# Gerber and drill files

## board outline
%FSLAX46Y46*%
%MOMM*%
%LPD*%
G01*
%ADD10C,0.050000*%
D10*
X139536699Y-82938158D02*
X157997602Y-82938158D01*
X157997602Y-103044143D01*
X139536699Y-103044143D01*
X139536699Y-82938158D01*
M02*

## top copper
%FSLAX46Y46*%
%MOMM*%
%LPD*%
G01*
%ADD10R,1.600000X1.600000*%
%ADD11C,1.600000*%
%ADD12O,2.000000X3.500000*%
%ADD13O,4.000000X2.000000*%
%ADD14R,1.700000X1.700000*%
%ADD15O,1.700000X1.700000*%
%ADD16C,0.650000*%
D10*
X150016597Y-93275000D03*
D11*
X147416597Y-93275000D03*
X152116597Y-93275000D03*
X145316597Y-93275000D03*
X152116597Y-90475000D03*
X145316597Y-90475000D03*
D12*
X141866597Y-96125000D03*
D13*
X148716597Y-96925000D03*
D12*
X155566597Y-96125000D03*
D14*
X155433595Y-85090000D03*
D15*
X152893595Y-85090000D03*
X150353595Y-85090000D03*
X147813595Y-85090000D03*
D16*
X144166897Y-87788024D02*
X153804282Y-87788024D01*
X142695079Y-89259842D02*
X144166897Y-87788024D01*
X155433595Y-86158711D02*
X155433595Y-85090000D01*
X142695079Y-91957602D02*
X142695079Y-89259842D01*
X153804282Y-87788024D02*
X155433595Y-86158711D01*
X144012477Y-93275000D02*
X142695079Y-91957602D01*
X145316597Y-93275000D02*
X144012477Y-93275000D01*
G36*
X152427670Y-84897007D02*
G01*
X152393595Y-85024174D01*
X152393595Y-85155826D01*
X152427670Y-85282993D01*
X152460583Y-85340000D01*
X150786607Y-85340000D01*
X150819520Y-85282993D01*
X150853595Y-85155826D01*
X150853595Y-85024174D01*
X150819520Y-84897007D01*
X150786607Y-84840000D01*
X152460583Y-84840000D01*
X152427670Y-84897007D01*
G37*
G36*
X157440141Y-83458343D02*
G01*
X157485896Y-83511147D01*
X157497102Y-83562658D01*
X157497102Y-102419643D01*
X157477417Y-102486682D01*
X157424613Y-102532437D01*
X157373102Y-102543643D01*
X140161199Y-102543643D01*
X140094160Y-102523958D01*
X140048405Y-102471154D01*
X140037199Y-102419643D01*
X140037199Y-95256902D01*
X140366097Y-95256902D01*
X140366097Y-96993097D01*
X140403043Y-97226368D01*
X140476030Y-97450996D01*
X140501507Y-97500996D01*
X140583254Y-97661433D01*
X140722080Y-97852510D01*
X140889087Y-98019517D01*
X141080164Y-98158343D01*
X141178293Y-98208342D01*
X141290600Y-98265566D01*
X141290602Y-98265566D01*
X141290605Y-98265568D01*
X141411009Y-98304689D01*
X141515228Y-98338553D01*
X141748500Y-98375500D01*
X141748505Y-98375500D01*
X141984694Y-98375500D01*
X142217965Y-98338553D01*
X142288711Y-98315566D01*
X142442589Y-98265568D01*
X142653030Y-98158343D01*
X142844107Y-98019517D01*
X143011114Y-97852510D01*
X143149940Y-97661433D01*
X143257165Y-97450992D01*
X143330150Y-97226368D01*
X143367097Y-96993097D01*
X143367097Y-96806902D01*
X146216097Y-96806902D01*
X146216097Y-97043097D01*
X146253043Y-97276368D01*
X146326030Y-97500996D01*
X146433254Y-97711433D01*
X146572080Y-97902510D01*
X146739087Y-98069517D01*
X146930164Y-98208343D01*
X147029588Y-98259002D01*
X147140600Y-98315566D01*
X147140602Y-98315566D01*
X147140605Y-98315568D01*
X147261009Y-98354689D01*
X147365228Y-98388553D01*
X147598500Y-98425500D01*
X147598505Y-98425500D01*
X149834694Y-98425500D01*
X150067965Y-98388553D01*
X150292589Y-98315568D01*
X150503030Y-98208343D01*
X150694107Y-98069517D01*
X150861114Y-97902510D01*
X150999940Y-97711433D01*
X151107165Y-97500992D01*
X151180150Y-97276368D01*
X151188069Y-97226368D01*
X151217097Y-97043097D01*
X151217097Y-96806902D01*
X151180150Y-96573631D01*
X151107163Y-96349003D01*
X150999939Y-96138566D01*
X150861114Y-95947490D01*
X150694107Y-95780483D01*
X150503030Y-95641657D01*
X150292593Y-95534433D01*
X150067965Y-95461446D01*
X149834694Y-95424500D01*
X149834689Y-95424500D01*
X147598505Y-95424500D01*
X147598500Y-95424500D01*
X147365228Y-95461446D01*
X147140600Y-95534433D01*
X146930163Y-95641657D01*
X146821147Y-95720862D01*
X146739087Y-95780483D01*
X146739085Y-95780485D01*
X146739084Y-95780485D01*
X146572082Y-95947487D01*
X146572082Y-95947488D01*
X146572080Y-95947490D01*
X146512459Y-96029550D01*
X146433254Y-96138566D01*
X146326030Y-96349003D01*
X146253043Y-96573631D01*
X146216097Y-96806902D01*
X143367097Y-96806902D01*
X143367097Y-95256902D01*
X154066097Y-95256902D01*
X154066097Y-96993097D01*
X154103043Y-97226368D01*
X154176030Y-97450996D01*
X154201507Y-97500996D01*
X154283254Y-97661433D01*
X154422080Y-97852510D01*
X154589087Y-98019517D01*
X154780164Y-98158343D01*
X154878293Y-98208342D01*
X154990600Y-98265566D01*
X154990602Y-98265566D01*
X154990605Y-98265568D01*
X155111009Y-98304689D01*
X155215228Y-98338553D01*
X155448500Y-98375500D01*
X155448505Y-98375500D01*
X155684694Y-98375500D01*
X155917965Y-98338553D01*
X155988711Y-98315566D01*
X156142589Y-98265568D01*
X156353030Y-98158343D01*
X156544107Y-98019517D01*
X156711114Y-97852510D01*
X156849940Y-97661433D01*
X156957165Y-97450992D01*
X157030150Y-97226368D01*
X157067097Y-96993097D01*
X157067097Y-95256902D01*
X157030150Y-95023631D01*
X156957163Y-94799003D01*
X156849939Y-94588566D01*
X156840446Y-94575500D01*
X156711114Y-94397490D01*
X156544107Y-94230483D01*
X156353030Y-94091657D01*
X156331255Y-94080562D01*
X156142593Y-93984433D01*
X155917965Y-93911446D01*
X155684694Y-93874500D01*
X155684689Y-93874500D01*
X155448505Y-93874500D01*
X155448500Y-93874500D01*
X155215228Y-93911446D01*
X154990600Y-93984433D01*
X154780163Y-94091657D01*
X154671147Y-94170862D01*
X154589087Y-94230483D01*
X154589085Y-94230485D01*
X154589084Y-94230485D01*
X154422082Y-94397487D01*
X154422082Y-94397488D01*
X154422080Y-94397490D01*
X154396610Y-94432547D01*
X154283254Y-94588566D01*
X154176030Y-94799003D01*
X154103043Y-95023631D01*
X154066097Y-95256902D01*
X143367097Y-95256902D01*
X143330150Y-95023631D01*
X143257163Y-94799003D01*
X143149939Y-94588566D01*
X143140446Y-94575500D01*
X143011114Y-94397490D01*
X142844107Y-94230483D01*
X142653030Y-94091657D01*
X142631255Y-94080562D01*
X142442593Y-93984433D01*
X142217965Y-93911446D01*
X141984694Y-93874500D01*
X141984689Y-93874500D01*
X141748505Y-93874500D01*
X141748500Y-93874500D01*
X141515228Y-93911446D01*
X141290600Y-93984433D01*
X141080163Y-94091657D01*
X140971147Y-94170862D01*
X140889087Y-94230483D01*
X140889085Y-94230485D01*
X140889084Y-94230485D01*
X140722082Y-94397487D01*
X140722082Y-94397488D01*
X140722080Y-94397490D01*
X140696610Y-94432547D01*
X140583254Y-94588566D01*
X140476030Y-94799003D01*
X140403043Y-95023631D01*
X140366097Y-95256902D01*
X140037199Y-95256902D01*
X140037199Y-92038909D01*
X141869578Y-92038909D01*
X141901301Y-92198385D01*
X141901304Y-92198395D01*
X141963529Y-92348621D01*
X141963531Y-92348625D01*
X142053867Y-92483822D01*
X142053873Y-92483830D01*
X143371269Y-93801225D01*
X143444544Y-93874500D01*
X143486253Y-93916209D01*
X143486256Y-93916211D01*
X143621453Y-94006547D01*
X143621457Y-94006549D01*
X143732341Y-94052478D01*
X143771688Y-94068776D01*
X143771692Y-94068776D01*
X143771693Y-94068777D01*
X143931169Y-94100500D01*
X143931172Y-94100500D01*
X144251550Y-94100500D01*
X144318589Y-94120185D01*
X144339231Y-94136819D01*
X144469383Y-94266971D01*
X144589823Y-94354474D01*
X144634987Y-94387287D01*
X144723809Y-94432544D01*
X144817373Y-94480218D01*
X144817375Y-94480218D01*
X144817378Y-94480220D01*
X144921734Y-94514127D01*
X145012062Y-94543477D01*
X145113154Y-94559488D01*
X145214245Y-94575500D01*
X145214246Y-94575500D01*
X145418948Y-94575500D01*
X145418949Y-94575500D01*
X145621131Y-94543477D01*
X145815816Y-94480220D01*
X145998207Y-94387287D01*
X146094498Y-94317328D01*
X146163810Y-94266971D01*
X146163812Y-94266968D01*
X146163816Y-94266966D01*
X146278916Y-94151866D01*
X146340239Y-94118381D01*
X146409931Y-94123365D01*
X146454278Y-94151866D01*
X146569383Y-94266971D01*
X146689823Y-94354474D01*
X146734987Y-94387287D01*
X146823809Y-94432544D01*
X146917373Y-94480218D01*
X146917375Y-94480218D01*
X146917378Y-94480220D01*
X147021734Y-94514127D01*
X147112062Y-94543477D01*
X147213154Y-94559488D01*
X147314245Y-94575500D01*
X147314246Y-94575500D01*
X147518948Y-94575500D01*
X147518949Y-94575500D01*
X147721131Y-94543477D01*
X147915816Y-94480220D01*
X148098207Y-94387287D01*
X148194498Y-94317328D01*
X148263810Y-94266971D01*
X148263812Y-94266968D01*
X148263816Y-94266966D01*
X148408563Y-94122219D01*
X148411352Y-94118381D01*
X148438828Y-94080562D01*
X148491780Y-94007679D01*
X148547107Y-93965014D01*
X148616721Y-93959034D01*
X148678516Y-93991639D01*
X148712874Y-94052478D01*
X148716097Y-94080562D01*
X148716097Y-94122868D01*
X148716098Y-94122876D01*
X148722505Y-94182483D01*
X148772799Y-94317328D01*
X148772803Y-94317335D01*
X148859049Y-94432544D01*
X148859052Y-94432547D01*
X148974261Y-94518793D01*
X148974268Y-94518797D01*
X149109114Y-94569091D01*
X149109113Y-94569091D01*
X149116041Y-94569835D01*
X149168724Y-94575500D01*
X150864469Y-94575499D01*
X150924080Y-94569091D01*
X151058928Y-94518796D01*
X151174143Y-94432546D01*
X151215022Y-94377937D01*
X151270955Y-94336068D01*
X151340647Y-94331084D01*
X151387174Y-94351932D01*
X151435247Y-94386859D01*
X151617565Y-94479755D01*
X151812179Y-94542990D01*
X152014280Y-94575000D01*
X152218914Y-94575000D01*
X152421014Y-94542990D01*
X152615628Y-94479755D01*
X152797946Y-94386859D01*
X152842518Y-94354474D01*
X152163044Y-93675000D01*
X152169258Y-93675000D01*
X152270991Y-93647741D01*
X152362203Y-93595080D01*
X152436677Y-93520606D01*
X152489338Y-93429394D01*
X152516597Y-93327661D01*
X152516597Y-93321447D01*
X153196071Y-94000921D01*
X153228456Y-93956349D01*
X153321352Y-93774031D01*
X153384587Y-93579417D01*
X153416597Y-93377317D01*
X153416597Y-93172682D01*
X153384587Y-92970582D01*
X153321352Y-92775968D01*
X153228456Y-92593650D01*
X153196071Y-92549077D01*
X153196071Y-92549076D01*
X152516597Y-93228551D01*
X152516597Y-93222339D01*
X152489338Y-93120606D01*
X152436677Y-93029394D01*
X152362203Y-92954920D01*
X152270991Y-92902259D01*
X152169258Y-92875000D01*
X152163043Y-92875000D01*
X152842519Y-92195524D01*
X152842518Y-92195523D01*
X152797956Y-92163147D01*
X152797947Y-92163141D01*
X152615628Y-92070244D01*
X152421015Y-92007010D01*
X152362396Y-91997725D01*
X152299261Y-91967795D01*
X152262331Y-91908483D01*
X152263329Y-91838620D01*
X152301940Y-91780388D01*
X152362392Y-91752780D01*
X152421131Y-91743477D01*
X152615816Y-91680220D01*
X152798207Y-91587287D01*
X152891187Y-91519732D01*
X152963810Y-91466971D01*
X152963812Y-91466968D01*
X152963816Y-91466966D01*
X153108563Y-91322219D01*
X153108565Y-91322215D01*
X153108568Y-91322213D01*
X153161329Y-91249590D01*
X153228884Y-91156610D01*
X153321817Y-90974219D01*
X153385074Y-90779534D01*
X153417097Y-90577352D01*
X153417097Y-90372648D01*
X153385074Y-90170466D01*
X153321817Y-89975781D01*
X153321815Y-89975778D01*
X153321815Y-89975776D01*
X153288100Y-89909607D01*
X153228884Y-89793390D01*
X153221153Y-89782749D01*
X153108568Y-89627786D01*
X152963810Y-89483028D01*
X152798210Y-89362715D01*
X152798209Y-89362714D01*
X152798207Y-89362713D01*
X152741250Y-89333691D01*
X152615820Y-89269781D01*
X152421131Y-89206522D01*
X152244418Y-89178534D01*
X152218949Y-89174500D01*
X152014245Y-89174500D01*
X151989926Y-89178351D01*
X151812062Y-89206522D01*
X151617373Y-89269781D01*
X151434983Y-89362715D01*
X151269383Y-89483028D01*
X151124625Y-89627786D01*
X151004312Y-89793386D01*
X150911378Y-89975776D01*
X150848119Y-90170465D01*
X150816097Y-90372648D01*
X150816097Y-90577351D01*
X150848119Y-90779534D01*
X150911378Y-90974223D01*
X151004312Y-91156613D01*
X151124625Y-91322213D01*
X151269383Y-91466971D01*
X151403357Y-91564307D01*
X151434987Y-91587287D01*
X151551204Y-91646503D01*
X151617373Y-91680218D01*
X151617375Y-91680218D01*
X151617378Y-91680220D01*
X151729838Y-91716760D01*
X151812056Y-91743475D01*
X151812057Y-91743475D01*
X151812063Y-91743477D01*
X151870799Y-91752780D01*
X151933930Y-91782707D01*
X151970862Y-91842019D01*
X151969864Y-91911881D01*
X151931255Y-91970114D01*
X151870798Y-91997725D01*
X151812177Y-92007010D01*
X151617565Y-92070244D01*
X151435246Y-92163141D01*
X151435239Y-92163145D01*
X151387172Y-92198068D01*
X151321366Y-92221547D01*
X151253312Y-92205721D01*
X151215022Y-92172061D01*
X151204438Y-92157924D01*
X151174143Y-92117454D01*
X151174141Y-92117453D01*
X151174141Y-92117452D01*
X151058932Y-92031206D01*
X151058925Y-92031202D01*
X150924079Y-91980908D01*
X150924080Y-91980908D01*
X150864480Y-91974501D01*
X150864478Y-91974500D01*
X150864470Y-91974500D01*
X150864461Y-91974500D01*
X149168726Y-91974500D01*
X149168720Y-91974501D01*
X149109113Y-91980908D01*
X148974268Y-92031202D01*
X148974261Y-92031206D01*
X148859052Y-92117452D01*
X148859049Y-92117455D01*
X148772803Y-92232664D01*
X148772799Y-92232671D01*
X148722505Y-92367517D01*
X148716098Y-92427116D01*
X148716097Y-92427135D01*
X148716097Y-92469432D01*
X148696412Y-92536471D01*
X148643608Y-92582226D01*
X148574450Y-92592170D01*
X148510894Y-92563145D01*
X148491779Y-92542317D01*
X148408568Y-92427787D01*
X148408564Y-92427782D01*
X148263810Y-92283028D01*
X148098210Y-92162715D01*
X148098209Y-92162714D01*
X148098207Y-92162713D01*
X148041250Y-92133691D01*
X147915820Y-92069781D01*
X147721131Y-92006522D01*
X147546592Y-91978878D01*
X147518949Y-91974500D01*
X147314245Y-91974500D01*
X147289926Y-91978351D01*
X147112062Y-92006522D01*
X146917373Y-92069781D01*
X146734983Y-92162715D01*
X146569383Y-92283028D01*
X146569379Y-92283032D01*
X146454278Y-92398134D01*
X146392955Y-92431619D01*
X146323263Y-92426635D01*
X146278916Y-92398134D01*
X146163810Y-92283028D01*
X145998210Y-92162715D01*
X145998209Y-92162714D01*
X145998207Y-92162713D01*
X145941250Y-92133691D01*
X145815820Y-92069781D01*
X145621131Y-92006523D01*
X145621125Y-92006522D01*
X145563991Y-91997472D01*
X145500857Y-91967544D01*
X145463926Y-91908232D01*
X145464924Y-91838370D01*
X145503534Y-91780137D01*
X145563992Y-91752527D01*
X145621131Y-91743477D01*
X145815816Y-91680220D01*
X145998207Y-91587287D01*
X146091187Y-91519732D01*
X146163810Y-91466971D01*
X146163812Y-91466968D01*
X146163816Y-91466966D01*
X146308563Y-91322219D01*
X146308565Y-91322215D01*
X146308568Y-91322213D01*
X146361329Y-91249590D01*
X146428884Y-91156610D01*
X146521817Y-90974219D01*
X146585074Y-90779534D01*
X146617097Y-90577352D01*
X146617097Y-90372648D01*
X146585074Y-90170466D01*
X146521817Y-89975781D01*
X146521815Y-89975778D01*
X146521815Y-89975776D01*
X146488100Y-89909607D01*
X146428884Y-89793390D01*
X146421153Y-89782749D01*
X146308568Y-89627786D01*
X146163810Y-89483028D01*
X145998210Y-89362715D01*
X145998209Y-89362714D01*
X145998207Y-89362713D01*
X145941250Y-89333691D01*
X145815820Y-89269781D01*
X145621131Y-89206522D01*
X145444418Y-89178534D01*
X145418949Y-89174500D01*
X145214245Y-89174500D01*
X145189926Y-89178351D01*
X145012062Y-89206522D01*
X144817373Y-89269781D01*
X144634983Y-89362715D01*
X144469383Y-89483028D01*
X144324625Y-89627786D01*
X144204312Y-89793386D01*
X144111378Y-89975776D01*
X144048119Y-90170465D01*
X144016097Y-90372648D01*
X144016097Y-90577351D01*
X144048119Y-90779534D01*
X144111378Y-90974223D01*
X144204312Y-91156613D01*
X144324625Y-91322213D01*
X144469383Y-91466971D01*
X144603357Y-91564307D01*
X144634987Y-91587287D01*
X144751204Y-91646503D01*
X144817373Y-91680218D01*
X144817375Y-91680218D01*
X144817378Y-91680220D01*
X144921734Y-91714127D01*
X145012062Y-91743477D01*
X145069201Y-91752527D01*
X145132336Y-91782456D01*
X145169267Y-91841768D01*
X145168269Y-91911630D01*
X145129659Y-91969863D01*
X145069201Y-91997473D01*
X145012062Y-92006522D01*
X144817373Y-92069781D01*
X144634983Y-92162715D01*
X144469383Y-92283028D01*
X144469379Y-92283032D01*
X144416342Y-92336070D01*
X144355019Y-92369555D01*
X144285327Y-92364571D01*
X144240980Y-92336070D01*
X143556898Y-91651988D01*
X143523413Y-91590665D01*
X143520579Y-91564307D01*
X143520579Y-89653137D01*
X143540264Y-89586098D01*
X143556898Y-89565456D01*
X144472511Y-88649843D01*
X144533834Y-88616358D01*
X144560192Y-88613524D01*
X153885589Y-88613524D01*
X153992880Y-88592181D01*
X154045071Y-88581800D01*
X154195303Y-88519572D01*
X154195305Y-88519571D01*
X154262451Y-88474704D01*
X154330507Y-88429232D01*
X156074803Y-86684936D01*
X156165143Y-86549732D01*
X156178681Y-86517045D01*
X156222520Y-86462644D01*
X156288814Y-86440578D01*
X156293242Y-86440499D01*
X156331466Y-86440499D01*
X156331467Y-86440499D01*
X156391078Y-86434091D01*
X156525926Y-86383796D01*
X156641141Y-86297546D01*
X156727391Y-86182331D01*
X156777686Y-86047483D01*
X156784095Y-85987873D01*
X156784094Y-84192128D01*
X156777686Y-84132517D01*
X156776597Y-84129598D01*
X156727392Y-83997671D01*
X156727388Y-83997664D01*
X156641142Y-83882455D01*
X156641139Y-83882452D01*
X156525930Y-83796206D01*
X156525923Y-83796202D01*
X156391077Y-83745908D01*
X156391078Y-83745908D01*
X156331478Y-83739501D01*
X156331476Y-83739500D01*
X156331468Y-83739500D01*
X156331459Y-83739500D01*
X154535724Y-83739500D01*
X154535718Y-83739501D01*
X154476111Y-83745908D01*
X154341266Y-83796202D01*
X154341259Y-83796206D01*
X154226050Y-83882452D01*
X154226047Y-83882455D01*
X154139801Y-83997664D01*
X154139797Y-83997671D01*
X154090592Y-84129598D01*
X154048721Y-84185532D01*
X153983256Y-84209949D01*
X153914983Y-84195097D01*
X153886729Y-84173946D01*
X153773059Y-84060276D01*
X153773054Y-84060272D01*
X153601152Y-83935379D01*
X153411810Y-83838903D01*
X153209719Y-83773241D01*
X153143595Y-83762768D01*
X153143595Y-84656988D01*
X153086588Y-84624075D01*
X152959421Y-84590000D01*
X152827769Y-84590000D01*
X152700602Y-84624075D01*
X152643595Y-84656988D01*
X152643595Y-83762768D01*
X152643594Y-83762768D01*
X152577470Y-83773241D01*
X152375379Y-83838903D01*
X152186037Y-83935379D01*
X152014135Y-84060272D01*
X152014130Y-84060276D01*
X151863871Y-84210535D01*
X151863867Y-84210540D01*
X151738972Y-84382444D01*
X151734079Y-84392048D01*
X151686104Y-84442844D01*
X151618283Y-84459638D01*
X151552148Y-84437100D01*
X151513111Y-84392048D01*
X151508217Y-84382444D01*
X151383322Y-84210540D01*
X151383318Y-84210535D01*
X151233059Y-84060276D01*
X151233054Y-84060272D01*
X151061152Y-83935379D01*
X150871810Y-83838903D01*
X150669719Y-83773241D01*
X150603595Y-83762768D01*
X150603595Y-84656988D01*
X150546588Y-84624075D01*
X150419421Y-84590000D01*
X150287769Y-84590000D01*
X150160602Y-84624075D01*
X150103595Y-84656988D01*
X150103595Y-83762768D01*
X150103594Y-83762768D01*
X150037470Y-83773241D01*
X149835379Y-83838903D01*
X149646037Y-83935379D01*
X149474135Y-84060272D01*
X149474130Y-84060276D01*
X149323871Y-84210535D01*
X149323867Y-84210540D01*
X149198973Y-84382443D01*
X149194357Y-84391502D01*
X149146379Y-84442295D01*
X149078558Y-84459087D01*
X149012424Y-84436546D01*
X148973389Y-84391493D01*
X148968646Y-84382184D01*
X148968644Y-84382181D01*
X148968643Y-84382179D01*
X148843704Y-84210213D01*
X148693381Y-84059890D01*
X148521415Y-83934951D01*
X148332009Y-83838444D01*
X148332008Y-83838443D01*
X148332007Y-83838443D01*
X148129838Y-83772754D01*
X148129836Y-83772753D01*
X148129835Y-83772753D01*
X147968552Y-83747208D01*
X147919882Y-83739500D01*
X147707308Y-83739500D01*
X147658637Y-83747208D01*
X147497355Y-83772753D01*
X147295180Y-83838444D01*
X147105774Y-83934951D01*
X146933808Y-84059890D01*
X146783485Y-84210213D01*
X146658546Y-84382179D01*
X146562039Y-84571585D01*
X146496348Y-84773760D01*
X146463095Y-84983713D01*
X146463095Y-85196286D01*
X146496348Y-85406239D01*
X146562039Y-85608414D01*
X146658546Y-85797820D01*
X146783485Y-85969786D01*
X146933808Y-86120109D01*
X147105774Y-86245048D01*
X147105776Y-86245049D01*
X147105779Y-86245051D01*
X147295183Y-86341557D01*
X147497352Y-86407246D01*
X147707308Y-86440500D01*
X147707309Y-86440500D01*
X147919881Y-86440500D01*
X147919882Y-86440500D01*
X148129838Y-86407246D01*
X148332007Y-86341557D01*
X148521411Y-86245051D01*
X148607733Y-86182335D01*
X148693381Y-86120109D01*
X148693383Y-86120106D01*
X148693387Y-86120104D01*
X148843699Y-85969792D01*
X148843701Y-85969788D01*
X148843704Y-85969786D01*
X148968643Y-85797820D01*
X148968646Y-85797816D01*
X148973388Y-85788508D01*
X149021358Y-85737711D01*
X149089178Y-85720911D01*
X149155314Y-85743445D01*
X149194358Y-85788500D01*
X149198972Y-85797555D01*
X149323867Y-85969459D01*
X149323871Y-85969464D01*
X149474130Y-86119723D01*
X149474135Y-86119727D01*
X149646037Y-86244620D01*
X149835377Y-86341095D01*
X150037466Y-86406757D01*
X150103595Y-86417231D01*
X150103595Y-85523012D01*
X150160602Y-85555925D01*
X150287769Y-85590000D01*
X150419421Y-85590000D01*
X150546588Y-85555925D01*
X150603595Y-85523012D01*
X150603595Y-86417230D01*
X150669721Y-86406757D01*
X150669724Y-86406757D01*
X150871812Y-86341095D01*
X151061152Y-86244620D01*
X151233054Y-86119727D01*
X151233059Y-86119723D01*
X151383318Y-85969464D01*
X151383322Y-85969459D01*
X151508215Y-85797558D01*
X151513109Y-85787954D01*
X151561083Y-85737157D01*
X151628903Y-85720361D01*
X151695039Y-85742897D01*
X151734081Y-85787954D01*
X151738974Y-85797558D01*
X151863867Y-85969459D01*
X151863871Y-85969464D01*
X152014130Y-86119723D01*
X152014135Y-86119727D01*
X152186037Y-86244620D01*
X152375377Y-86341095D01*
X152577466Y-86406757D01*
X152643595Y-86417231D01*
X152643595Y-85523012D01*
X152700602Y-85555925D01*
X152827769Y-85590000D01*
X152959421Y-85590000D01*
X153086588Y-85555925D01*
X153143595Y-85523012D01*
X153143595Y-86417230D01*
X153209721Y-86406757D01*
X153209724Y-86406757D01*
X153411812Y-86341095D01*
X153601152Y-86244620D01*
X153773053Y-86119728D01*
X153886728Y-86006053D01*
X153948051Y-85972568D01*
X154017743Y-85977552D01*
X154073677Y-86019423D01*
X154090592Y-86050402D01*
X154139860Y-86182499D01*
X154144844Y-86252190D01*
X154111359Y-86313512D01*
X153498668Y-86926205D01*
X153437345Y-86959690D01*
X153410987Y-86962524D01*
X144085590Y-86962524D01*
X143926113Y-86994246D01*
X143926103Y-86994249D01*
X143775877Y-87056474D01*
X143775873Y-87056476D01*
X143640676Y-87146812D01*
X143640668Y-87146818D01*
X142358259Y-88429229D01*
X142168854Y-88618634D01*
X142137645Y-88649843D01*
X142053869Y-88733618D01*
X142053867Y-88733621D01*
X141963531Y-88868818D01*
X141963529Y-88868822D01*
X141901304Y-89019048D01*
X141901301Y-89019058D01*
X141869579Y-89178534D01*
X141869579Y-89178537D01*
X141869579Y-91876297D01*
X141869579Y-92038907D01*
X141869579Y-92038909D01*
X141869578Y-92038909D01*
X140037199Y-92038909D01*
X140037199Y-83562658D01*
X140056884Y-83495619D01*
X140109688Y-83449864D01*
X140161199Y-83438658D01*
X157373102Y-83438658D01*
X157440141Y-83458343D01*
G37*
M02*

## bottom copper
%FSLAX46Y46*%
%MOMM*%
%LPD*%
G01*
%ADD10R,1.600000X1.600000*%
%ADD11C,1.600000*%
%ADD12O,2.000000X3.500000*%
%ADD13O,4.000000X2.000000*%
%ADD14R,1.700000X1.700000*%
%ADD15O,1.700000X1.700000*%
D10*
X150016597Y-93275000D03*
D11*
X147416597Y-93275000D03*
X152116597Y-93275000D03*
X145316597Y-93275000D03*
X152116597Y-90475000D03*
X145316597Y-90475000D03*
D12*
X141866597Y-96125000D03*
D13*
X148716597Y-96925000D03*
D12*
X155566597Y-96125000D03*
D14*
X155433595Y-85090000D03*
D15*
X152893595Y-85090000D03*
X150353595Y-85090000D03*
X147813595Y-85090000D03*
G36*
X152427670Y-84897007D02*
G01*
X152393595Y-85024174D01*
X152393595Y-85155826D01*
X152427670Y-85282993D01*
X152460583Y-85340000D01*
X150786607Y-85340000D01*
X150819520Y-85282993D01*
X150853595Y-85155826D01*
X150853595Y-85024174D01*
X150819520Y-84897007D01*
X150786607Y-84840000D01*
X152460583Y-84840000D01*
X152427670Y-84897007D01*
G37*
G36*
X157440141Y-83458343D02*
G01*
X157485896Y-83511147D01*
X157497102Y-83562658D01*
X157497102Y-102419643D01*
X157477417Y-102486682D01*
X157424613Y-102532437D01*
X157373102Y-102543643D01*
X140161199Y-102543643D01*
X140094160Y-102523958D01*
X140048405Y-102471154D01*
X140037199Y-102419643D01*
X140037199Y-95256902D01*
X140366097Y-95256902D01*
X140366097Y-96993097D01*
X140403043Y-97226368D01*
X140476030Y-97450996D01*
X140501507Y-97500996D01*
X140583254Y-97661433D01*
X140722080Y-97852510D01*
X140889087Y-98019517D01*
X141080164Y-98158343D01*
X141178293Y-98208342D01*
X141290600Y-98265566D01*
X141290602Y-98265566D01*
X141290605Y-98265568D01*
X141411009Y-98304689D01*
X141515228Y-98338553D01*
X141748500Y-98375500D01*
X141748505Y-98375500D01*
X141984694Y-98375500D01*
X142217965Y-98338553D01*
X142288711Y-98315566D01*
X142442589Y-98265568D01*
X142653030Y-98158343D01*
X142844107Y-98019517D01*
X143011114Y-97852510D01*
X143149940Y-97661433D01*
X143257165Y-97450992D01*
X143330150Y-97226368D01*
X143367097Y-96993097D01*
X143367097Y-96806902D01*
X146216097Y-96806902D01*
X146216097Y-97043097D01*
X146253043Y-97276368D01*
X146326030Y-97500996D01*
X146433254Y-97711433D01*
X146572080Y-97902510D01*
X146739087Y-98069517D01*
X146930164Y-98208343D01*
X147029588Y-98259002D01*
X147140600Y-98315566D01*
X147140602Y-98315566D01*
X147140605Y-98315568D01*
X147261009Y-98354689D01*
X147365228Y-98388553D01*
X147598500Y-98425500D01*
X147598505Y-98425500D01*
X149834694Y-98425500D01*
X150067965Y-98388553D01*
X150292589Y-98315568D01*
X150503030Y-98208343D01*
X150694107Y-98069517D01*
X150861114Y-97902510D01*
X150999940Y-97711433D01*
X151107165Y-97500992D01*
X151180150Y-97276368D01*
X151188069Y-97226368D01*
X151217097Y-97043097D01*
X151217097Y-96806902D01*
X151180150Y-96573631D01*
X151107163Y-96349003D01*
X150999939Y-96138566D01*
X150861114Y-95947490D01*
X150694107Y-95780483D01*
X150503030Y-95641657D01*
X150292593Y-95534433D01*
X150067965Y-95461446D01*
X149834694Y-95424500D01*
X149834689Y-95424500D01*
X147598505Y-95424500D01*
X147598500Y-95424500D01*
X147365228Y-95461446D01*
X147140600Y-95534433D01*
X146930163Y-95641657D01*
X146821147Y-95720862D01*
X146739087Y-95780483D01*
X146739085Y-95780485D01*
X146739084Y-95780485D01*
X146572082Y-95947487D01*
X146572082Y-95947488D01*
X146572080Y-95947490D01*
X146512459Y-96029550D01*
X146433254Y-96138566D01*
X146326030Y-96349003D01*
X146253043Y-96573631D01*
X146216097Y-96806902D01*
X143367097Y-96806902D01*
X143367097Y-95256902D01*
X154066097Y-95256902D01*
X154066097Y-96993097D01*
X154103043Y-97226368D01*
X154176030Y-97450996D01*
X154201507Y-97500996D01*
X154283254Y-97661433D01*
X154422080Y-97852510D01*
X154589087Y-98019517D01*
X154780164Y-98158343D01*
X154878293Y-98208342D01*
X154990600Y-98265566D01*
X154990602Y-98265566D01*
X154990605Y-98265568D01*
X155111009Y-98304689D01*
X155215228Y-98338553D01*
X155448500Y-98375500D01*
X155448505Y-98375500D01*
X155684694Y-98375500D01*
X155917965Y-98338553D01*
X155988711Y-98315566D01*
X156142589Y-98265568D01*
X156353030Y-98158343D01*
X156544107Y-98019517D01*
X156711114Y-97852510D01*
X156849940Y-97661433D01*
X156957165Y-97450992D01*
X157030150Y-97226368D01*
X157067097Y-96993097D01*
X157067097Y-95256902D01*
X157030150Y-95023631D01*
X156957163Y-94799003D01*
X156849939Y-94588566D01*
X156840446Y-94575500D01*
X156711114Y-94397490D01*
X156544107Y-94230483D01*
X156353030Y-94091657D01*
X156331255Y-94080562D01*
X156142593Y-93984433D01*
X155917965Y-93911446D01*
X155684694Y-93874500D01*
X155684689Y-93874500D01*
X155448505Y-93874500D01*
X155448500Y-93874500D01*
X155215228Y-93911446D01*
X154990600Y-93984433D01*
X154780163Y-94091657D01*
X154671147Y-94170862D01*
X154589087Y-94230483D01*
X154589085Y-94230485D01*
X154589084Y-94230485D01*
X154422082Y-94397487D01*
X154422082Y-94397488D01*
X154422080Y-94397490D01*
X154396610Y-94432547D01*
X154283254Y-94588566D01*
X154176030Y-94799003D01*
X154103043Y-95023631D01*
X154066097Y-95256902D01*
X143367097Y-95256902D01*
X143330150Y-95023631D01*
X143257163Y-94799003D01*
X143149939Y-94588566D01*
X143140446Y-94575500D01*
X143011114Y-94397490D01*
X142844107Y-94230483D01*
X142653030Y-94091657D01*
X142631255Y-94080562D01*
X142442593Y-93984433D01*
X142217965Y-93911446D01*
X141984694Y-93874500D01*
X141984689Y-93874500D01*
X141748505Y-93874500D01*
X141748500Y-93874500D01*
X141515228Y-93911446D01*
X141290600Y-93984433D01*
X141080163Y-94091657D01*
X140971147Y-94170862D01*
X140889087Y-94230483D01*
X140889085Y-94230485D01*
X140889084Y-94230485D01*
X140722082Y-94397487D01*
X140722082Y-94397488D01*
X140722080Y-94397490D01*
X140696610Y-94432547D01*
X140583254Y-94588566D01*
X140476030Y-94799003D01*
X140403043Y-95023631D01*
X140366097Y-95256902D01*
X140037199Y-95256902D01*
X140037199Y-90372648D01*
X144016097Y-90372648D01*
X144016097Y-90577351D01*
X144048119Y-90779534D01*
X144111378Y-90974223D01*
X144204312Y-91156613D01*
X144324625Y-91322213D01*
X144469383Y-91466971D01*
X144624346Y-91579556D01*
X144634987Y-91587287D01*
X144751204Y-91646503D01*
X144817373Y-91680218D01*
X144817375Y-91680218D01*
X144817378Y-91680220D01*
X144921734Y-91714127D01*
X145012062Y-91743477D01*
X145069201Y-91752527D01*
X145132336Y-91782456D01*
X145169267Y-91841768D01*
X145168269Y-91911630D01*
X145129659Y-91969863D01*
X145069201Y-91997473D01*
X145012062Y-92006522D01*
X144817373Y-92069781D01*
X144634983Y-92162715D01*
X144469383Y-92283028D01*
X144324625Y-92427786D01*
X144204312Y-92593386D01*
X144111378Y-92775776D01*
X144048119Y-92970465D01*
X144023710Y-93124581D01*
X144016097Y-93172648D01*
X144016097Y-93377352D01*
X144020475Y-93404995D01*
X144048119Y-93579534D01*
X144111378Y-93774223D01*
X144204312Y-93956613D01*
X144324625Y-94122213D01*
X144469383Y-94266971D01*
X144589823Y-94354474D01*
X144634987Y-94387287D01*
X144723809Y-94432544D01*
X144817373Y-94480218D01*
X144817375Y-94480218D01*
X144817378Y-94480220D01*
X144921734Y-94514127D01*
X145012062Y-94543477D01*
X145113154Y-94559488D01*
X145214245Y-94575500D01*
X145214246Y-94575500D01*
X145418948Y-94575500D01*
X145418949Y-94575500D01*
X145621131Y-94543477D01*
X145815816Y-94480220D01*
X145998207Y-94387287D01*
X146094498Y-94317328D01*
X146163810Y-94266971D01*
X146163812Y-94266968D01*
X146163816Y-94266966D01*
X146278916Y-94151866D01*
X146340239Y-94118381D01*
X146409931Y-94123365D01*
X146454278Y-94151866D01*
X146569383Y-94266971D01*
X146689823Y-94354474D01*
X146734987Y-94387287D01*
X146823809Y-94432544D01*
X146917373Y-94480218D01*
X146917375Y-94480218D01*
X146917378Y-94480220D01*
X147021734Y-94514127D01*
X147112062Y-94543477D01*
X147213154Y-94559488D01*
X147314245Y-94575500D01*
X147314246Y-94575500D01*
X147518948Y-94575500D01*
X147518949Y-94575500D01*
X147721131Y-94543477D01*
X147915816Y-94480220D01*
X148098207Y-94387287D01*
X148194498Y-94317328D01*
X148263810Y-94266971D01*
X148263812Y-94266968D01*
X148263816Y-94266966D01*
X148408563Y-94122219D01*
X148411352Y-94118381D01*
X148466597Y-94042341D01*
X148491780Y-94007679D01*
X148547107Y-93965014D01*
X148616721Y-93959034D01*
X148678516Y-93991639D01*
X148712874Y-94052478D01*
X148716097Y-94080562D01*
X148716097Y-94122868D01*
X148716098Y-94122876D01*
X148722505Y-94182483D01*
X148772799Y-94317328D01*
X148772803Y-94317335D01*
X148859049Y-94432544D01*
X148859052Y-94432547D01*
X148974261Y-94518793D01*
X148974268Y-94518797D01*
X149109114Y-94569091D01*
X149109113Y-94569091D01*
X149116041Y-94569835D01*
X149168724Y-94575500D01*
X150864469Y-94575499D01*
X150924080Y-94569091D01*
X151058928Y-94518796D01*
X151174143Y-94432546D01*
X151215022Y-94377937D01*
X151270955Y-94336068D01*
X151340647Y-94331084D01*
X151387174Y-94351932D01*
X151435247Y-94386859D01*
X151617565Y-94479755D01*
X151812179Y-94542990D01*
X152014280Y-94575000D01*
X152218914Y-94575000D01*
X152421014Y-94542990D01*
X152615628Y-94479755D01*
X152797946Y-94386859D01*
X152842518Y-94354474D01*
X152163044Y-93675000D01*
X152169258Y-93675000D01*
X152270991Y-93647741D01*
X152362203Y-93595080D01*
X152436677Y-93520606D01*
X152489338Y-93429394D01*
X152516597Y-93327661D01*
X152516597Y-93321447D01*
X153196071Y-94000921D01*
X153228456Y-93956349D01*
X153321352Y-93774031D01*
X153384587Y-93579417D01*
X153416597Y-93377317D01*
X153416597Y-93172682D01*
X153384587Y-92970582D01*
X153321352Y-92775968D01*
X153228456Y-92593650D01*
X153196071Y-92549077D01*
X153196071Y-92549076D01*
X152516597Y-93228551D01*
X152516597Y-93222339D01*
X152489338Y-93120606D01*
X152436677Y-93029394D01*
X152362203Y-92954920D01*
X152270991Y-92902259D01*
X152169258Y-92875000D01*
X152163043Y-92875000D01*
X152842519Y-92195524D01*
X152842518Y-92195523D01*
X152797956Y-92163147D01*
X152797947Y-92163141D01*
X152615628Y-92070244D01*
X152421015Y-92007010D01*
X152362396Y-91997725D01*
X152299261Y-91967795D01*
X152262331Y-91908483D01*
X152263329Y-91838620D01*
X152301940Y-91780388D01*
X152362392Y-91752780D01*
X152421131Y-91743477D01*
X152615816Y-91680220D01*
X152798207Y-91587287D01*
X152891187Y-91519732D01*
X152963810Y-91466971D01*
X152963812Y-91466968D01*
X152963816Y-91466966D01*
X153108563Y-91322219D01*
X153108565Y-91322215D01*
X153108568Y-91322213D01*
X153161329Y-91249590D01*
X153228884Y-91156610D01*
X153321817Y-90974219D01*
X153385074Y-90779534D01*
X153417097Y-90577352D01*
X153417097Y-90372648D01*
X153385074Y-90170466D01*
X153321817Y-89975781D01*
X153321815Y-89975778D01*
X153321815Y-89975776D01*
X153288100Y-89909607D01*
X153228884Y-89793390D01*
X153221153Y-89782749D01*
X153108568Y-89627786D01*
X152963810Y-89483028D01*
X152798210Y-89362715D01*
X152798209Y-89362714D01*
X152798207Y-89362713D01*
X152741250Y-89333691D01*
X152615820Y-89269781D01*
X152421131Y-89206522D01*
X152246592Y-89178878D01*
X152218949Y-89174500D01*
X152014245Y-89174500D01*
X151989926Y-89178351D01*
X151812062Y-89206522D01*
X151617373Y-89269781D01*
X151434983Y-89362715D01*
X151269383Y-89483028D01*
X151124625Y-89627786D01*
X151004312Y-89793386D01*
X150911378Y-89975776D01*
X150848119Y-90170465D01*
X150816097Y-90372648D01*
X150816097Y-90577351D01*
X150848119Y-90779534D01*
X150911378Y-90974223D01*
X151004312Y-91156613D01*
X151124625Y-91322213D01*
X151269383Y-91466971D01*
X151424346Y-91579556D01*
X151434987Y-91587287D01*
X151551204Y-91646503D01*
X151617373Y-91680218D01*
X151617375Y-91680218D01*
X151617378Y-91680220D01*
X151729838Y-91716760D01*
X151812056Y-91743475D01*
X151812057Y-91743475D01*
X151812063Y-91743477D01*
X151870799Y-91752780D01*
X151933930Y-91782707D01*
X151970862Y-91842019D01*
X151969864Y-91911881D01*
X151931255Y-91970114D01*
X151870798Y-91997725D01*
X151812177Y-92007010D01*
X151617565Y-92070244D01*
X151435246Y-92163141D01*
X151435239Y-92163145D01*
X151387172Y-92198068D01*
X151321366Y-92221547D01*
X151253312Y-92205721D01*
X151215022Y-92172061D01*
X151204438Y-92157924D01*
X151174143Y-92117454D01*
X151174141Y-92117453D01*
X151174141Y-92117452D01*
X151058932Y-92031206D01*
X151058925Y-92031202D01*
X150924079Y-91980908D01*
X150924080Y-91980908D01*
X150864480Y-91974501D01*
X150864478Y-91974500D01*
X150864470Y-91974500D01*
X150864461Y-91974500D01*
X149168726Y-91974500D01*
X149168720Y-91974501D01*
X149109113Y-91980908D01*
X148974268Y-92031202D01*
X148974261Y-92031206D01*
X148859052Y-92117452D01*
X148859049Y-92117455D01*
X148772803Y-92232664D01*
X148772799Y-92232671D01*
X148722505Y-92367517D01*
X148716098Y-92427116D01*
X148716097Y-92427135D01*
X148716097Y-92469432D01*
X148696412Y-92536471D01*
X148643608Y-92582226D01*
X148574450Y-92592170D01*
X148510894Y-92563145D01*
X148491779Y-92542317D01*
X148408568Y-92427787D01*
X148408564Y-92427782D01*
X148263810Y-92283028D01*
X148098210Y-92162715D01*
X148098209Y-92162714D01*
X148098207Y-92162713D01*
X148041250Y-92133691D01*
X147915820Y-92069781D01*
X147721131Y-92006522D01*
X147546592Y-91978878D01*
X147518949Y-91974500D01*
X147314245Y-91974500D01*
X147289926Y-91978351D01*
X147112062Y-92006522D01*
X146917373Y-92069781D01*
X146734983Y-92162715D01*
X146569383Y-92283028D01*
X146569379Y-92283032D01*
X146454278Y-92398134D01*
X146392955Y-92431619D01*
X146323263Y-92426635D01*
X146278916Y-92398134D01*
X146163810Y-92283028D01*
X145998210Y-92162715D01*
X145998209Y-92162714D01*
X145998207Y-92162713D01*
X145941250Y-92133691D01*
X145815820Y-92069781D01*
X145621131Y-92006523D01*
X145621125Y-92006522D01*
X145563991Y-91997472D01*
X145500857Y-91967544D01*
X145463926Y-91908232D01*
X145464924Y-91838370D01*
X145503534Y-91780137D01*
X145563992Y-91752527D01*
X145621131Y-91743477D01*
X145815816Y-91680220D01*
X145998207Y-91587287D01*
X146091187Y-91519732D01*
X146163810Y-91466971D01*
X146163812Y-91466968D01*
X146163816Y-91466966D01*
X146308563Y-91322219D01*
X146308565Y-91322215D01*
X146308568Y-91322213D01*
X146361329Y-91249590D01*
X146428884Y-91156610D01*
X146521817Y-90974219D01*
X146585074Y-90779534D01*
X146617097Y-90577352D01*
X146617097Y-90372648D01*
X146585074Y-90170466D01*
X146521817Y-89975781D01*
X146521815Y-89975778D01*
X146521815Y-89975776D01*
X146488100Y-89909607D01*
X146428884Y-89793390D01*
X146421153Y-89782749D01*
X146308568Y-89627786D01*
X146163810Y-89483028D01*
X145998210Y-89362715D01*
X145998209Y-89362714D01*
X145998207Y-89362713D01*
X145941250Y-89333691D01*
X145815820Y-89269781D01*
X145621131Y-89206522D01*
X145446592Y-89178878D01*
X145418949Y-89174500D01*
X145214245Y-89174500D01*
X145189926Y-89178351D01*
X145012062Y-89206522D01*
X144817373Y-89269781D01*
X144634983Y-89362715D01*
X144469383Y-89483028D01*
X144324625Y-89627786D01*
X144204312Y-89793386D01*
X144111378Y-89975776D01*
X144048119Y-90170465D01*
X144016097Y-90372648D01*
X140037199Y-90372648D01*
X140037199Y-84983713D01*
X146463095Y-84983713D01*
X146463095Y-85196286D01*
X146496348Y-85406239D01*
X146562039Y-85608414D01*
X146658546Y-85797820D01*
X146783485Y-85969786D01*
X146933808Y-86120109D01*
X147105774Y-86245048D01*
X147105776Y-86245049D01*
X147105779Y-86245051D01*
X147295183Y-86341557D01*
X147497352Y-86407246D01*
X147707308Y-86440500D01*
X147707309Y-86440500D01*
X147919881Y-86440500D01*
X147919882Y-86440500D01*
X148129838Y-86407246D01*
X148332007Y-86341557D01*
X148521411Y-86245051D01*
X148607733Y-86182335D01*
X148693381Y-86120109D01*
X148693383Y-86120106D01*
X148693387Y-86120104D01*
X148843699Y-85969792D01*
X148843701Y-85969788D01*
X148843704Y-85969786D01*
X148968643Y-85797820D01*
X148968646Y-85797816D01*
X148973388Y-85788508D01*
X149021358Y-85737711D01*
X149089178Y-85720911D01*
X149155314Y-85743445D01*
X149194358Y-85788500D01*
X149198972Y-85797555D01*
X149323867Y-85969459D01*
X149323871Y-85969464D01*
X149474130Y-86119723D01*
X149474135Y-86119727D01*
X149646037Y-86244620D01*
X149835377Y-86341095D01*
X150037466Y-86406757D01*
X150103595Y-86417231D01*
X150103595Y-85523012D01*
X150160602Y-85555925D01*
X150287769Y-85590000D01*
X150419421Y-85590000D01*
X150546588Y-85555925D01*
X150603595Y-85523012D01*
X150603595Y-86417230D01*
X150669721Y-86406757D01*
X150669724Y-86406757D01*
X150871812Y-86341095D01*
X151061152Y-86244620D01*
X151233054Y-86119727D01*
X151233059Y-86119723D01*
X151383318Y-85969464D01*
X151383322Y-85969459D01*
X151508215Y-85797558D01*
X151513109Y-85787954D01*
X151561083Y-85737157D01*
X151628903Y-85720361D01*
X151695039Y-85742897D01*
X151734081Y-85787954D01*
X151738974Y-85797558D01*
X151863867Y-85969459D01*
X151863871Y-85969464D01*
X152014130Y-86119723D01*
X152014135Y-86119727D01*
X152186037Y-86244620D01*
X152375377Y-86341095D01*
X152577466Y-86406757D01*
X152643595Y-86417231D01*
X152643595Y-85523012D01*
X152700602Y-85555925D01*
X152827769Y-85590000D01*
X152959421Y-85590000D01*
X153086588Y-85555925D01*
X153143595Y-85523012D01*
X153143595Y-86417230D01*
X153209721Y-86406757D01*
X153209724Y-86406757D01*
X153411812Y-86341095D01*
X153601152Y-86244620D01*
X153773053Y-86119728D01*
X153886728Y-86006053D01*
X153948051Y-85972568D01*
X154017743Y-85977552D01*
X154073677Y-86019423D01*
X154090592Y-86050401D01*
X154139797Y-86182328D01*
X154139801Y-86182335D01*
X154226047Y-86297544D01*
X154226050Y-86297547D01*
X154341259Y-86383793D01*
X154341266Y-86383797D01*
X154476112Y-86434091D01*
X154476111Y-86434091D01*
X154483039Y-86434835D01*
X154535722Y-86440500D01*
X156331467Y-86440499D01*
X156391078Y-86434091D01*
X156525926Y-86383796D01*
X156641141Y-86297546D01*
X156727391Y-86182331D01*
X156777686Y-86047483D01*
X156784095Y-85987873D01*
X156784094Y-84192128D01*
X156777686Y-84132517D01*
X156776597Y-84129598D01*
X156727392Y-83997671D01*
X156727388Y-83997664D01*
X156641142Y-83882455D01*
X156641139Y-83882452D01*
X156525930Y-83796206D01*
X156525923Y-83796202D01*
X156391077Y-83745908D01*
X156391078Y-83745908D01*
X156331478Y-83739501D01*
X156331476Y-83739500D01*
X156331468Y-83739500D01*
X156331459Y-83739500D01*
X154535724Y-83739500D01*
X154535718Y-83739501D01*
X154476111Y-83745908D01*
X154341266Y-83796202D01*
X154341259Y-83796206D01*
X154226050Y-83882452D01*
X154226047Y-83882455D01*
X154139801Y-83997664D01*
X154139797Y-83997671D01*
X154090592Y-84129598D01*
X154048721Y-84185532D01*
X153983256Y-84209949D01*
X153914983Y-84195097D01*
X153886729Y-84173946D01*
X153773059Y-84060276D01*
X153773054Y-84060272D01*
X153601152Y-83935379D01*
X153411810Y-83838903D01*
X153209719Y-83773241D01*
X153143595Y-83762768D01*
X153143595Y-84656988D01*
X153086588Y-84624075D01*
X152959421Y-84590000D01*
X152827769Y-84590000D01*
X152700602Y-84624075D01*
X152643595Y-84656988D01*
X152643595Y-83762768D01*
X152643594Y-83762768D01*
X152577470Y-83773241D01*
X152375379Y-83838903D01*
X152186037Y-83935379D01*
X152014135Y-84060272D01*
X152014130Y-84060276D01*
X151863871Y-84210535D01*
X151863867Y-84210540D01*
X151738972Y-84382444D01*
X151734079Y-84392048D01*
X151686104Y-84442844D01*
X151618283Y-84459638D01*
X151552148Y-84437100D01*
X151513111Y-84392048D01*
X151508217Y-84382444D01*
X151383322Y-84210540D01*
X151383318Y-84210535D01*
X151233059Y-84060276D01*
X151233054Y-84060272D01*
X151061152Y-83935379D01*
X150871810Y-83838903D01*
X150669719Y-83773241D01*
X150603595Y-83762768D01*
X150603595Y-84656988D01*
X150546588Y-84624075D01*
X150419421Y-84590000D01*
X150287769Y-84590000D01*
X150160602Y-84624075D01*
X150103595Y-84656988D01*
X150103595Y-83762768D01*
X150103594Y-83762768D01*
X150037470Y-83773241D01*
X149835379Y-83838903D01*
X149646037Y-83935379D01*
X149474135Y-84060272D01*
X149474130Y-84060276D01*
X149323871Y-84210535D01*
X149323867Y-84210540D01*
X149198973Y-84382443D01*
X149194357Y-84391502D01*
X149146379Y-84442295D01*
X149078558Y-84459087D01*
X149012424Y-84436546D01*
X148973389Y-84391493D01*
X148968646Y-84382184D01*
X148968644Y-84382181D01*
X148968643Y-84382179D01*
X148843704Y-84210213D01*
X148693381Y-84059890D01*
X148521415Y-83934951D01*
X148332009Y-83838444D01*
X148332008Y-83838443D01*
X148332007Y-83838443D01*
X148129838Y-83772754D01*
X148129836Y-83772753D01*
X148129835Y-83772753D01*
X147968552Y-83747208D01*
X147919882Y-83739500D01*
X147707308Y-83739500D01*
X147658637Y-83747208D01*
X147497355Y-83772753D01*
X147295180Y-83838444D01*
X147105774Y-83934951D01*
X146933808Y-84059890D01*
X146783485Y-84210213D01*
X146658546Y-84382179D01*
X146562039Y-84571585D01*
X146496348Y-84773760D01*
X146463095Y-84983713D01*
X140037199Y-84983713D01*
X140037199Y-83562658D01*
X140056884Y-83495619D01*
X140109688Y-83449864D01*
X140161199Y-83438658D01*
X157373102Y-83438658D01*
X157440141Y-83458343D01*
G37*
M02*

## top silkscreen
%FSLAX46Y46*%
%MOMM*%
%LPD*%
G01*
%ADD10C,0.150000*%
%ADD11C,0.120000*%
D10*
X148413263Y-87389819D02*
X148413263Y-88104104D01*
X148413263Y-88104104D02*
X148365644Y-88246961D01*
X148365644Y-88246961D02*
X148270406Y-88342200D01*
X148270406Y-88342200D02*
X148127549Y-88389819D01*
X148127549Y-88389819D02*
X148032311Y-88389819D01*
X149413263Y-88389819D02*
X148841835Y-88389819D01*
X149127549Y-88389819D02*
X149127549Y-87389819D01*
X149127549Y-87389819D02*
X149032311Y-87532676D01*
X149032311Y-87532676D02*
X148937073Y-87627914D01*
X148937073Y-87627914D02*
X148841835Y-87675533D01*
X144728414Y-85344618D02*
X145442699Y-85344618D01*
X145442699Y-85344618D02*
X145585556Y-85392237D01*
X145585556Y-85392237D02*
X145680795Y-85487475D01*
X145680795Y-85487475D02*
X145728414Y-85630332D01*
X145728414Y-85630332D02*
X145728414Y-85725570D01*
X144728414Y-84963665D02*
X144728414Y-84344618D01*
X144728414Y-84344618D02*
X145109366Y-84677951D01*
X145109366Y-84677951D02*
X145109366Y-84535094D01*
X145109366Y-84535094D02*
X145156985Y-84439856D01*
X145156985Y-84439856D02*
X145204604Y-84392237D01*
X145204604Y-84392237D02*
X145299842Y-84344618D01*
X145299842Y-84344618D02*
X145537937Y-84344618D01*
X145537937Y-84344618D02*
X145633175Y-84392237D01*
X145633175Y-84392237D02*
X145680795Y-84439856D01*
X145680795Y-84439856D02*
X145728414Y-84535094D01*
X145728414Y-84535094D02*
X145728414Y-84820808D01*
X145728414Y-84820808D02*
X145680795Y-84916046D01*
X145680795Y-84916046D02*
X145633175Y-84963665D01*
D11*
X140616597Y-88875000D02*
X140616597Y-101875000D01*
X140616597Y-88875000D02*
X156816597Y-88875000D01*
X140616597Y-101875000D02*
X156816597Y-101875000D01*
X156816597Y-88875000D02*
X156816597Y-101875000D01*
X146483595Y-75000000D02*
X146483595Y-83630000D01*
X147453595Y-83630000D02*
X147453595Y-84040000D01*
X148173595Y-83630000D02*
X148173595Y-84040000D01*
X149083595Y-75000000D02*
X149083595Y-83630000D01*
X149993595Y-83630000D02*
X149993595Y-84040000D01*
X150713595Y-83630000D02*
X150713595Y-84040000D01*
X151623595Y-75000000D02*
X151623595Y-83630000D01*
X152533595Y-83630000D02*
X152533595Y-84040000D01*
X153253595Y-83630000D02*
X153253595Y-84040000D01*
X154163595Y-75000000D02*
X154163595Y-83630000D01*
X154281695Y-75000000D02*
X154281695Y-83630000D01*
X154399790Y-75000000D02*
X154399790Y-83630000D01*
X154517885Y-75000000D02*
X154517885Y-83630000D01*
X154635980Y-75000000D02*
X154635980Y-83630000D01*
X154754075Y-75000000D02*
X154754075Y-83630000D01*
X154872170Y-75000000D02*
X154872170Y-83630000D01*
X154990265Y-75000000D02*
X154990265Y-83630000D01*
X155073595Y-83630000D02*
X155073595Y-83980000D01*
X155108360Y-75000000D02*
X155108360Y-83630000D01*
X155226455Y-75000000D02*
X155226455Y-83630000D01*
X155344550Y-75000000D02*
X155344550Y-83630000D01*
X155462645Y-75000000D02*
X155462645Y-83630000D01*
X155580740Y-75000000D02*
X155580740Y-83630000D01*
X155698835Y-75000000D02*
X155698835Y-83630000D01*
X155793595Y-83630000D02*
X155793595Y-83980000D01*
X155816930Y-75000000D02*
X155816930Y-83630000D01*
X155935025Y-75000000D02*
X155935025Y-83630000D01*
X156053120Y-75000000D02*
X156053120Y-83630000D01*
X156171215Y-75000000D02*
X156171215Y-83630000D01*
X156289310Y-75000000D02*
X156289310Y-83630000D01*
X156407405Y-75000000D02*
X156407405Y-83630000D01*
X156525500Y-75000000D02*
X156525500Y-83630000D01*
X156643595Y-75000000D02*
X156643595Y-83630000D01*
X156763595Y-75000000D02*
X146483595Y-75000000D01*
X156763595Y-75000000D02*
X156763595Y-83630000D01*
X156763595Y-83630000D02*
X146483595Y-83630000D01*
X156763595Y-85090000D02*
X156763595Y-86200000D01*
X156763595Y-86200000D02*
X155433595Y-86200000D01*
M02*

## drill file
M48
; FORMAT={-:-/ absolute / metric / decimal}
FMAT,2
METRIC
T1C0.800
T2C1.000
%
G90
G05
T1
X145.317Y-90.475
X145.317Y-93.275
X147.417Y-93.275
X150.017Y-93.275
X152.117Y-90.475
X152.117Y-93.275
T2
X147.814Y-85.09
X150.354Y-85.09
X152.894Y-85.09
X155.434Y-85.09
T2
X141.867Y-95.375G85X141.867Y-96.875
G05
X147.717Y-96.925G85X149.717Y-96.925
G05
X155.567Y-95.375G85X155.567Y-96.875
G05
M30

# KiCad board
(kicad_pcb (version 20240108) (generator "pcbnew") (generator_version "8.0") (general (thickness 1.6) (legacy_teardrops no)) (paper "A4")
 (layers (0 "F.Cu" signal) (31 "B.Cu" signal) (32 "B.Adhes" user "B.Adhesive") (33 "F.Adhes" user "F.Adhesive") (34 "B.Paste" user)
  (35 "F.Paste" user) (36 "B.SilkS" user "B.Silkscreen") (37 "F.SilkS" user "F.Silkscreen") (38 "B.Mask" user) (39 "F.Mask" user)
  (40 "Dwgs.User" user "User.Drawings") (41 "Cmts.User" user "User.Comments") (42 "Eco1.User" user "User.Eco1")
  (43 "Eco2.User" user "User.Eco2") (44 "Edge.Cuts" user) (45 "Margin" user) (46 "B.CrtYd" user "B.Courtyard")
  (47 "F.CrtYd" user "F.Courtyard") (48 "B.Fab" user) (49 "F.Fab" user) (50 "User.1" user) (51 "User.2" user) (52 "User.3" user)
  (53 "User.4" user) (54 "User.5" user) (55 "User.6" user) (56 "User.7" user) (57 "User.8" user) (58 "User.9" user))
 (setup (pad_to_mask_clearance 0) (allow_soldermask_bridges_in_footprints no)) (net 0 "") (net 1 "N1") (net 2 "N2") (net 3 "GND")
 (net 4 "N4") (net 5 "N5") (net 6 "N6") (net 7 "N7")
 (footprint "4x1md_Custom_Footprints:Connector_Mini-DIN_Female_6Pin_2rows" (layer "F.Cu") (at 150.016597 93.275)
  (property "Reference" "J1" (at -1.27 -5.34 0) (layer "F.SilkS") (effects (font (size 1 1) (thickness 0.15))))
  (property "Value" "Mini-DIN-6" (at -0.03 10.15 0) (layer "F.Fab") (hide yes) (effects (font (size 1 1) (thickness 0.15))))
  (fp_line (start -9.4 -4.4) (end -9.4 8.6) (stroke (width 0.12) (type solid)) (layer "F.SilkS"))
  (fp_line (start -9.4 -4.4) (end 6.8 -4.4) (stroke (width 0.12) (type solid)) (layer "F.SilkS"))
  (fp_line (start -9.4 8.6) (end 6.8 8.6) (stroke (width 0.12) (type solid)) (layer "F.SilkS"))
  (fp_line (start 6.8 -4.4) (end 6.8 8.6) (stroke (width 0.12) (type solid)) (layer "F.SilkS"))
  (pad "1" thru_hole rect (at 0 0) (size 1.6 1.6) (drill 0.8) (layers "*.Cu" "*.Mask") (remove_unused_layers no) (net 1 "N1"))
  (pad "2" thru_hole circle (at -2.6 0) (size 1.6 1.6) (drill 0.8) (layers "*.Cu" "*.Mask") (remove_unused_layers no) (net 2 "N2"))
  (pad "3" thru_hole circle (at 2.1 0) (size 1.6 1.6) (drill 0.8) (layers "*.Cu" "*.Mask") (remove_unused_layers no) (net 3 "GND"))
  (pad "4" thru_hole circle (at -4.7 0) (size 1.6 1.6) (drill 0.8) (layers "*.Cu" "*.Mask") (remove_unused_layers no) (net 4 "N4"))
  (pad "5" thru_hole circle (at 2.1 -2.8) (size 1.6 1.6) (drill 0.8) (layers "*.Cu" "*.Mask") (remove_unused_layers no) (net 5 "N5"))
  (pad "6" thru_hole circle (at -4.7 -2.8) (size 1.6 1.6) (drill 0.8) (layers "*.Cu" "*.Mask") (remove_unused_layers no) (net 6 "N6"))
  (pad "7" thru_hole oval (at -8.15 2.85) (size 2 3.5) (drill oval 1 2.5) (layers "*.Cu" "*.Mask") (remove_unused_layers no))
  (pad "7" thru_hole oval (at -1.3 3.65) (size 4 2) (drill oval 3 1) (layers "*.Cu" "*.Mask") (remove_unused_layers no))
  (pad "7" thru_hole oval (at 5.55 2.85) (size 2 3.5) (drill oval 1 2.5) (layers "*.Cu" "*.Mask") (remove_unused_layers no)))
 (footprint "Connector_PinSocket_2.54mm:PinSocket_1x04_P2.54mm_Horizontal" (layer "F.Cu") (at 155.433595 85.09 -90)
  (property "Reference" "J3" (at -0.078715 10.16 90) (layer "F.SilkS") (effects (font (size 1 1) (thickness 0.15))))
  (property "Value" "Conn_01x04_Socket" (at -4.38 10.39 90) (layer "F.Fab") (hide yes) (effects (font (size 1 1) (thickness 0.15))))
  (fp_line (start -10.09 8.95) (end -1.46 8.95) (stroke (width 0.12) (type solid)) (layer "F.SilkS"))
  (fp_line (start -1.46 7.98) (end -1.05 7.98) (stroke (width 0.12) (type solid)) (layer "F.SilkS"))
  (fp_line (start -1.46 7.26) (end -1.05 7.26) (stroke (width 0.12) (type solid)) (layer "F.SilkS"))
  (fp_line (start -10.09 6.35) (end -1.46 6.35) (stroke (width 0.12) (type solid)) (layer "F.SilkS"))
  (fp_line (start -1.46 5.44) (end -1.05 5.44) (stroke (width 0.12) (type solid)) (layer "F.SilkS"))
  (fp_line (start -1.46 4.72) (end -1.05 4.72) (stroke (width 0.12) (type solid)) (layer "F.SilkS"))
  (fp_line (start -10.09 3.81) (end -1.46 3.81) (stroke (width 0.12) (type solid)) (layer "F.SilkS"))
  (fp_line (start -1.46 2.9) (end -1.05 2.9) (stroke (width 0.12) (type solid)) (layer "F.SilkS"))
  (fp_line (start -1.46 2.18) (end -1.05 2.18) (stroke (width 0.12) (type solid)) (layer "F.SilkS"))
  (fp_line (start -10.09 1.27) (end -1.46 1.27) (stroke (width 0.12) (type solid)) (layer "F.SilkS"))
  (fp_line (start -10.09 1.1519) (end -1.46 1.1519) (stroke (width 0.12) (type solid)) (layer "F.SilkS"))
  (fp_line (start -10.09 1.033805) (end -1.46 1.033805) (stroke (width 0.12) (type solid)) (layer "F.SilkS"))
  (fp_line (start -10.09 0.91571) (end -1.46 0.91571) (stroke (width 0.12) (type solid)) (layer "F.SilkS"))
  (fp_line (start -10.09 0.797615) (end -1.46 0.797615) (stroke (width 0.12) (type solid)) (layer "F.SilkS"))
  (fp_line (start -10.09 0.67952) (end -1.46 0.67952) (stroke (width 0.12) (type solid)) (layer "F.SilkS"))
  (fp_line (start -10.09 0.561425) (end -1.46 0.561425) (stroke (width 0.12) (type solid)) (layer "F.SilkS"))
  (fp_line (start -10.09 0.44333) (end -1.46 0.44333) (stroke (width 0.12) (type solid)) (layer "F.SilkS"))
  (fp_line (start -1.46 0.36) (end -1.11 0.36) (stroke (width 0.12) (type solid)) (layer "F.SilkS"))
  (fp_line (start -10.09 0.325235) (end -1.46 0.325235) (stroke (width 0.12) (type solid)) (layer "F.SilkS"))
  (fp_line (start -10.09 0.20714) (end -1.46 0.20714) (stroke (width 0.12) (type solid)) (layer "F.SilkS"))
  (fp_line (start -10.09 0.089045) (end -1.46 0.089045) (stroke (width 0.12) (type solid)) (layer "F.SilkS"))
  (fp_line (start -10.09 -0.02905) (end -1.46 -0.02905) (stroke (width 0.12) (type solid)) (layer "F.SilkS"))
  (fp_line (start -10.09 -0.147145) (end -1.46 -0.147145) (stroke (width 0.12) (type solid)) (layer "F.SilkS"))
  (fp_line (start -10.09 -0.26524) (end -1.46 -0.26524) (stroke (width 0.12) (type solid)) (layer "F.SilkS"))
  (fp_line (start -1.46 -0.36) (end -1.11 -0.36) (stroke (width 0.12) (type solid)) (layer "F.SilkS"))
  (fp_line (start -10.09 -0.383335) (end -1.46 -0.383335) (stroke (width 0.12) (type solid)) (layer "F.SilkS"))
  (fp_line (start -10.09 -0.50143) (end -1.46 -0.50143) (stroke (width 0.12) (type solid)) (layer "F.SilkS"))
  (fp_line (start -10.09 -0.619525) (end -1.46 -0.619525) (stroke (width 0.12) (type solid)) (layer "F.SilkS"))
  (fp_line (start -10.09 -0.73762) (end -1.46 -0.73762) (stroke (width 0.12) (type solid)) (layer "F.SilkS"))
  (fp_line (start -10.09 -0.855715) (end -1.46 -0.855715) (stroke (width 0.12) (type solid)) (layer "F.SilkS"))
  (fp_line (start -10.09 -0.97381) (end -1.46 -0.97381) (stroke (width 0.12) (type solid)) (layer "F.SilkS"))
  (fp_line (start -10.09 -1.091905) (end -1.46 -1.091905) (stroke (width 0.12) (type solid)) (layer "F.SilkS"))
  (fp_line (start -10.09 -1.21) (end -1.46 -1.21) (stroke (width 0.12) (type solid)) (layer "F.SilkS"))
  (fp_line (start -10.09 -1.33) (end -10.09 8.95) (stroke (width 0.12) (type solid)) (layer "F.SilkS"))
  (fp_line (start -10.09 -1.33) (end -1.46 -1.33) (stroke (width 0.12) (type solid)) (layer "F.SilkS"))
  (fp_line (start -1.46 -1.33) (end -1.46 8.95) (stroke (width 0.12) (type solid)) (layer "F.SilkS"))
  (fp_line (start 0 -1.33) (end 1.11 -1.33) (stroke (width 0.12) (type solid)) (layer "F.SilkS"))
  (fp_line (start 1.11 -1.33) (end 1.11 0) (stroke (width 0.12) (type solid)) (layer "F.SilkS"))
  (pad "1" thru_hole rect (at 0 0 270) (size 1.7 1.7) (drill 1) (layers "*.Cu" "*.Mask") (remove_unused_layers no) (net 4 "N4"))
  (pad "2" thru_hole oval (at 0 2.54 270) (size 1.7 1.7) (drill 1) (layers "*.Cu" "*.Mask") (remove_unused_layers no) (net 3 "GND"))
  (pad "3" thru_hole oval (at 0 5.08 270) (size 1.7 1.7) (drill 1) (layers "*.Cu" "*.Mask") (remove_unused_layers no) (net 3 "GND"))
  (pad "4" thru_hole oval (at 0 7.62 270) (size 1.7 1.7) (drill 1) (layers "*.Cu" "*.Mask") (remove_unused_layers no) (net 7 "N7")))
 (gr_rect (start 139.536699 82.938158) (end 157.997602 103.044143) (stroke (width 0.05) (type default)) (fill none) (layer "Edge.Cuts"))
 (segment (start 144.166897 87.788024) (end 153.804282 87.788024) (width 0.65) (layer "F.Cu") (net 4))
 (segment (start 142.695079 89.259842) (end 144.166897 87.788024) (width 0.65) (layer "F.Cu") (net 4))
 (segment (start 155.433595 86.158711) (end 155.433595 85.09) (width 0.65) (layer "F.Cu") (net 4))
 (segment (start 142.695079 91.957602) (end 142.695079 89.259842) (width 0.65) (layer "F.Cu") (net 4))
 (segment (start 153.804282 87.788024) (end 155.433595 86.158711) (width 0.65) (layer "F.Cu") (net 4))
 (segment (start 144.012477 93.275) (end 142.695079 91.957602) (width 0.65) (layer "F.Cu") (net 4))
 (segment (start 145.316597 93.275) (end 144.012477 93.275) (width 0.65) (layer "F.Cu") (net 4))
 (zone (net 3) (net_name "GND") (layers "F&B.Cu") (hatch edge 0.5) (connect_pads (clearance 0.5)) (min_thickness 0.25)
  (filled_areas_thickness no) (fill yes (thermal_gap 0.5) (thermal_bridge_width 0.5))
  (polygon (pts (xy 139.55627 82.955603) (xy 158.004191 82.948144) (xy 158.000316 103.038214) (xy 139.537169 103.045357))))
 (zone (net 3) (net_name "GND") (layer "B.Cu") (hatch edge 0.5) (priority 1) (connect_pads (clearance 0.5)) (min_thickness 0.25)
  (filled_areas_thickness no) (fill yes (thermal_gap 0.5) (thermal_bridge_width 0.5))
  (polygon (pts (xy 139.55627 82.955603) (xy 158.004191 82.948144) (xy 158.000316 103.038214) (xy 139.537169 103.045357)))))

